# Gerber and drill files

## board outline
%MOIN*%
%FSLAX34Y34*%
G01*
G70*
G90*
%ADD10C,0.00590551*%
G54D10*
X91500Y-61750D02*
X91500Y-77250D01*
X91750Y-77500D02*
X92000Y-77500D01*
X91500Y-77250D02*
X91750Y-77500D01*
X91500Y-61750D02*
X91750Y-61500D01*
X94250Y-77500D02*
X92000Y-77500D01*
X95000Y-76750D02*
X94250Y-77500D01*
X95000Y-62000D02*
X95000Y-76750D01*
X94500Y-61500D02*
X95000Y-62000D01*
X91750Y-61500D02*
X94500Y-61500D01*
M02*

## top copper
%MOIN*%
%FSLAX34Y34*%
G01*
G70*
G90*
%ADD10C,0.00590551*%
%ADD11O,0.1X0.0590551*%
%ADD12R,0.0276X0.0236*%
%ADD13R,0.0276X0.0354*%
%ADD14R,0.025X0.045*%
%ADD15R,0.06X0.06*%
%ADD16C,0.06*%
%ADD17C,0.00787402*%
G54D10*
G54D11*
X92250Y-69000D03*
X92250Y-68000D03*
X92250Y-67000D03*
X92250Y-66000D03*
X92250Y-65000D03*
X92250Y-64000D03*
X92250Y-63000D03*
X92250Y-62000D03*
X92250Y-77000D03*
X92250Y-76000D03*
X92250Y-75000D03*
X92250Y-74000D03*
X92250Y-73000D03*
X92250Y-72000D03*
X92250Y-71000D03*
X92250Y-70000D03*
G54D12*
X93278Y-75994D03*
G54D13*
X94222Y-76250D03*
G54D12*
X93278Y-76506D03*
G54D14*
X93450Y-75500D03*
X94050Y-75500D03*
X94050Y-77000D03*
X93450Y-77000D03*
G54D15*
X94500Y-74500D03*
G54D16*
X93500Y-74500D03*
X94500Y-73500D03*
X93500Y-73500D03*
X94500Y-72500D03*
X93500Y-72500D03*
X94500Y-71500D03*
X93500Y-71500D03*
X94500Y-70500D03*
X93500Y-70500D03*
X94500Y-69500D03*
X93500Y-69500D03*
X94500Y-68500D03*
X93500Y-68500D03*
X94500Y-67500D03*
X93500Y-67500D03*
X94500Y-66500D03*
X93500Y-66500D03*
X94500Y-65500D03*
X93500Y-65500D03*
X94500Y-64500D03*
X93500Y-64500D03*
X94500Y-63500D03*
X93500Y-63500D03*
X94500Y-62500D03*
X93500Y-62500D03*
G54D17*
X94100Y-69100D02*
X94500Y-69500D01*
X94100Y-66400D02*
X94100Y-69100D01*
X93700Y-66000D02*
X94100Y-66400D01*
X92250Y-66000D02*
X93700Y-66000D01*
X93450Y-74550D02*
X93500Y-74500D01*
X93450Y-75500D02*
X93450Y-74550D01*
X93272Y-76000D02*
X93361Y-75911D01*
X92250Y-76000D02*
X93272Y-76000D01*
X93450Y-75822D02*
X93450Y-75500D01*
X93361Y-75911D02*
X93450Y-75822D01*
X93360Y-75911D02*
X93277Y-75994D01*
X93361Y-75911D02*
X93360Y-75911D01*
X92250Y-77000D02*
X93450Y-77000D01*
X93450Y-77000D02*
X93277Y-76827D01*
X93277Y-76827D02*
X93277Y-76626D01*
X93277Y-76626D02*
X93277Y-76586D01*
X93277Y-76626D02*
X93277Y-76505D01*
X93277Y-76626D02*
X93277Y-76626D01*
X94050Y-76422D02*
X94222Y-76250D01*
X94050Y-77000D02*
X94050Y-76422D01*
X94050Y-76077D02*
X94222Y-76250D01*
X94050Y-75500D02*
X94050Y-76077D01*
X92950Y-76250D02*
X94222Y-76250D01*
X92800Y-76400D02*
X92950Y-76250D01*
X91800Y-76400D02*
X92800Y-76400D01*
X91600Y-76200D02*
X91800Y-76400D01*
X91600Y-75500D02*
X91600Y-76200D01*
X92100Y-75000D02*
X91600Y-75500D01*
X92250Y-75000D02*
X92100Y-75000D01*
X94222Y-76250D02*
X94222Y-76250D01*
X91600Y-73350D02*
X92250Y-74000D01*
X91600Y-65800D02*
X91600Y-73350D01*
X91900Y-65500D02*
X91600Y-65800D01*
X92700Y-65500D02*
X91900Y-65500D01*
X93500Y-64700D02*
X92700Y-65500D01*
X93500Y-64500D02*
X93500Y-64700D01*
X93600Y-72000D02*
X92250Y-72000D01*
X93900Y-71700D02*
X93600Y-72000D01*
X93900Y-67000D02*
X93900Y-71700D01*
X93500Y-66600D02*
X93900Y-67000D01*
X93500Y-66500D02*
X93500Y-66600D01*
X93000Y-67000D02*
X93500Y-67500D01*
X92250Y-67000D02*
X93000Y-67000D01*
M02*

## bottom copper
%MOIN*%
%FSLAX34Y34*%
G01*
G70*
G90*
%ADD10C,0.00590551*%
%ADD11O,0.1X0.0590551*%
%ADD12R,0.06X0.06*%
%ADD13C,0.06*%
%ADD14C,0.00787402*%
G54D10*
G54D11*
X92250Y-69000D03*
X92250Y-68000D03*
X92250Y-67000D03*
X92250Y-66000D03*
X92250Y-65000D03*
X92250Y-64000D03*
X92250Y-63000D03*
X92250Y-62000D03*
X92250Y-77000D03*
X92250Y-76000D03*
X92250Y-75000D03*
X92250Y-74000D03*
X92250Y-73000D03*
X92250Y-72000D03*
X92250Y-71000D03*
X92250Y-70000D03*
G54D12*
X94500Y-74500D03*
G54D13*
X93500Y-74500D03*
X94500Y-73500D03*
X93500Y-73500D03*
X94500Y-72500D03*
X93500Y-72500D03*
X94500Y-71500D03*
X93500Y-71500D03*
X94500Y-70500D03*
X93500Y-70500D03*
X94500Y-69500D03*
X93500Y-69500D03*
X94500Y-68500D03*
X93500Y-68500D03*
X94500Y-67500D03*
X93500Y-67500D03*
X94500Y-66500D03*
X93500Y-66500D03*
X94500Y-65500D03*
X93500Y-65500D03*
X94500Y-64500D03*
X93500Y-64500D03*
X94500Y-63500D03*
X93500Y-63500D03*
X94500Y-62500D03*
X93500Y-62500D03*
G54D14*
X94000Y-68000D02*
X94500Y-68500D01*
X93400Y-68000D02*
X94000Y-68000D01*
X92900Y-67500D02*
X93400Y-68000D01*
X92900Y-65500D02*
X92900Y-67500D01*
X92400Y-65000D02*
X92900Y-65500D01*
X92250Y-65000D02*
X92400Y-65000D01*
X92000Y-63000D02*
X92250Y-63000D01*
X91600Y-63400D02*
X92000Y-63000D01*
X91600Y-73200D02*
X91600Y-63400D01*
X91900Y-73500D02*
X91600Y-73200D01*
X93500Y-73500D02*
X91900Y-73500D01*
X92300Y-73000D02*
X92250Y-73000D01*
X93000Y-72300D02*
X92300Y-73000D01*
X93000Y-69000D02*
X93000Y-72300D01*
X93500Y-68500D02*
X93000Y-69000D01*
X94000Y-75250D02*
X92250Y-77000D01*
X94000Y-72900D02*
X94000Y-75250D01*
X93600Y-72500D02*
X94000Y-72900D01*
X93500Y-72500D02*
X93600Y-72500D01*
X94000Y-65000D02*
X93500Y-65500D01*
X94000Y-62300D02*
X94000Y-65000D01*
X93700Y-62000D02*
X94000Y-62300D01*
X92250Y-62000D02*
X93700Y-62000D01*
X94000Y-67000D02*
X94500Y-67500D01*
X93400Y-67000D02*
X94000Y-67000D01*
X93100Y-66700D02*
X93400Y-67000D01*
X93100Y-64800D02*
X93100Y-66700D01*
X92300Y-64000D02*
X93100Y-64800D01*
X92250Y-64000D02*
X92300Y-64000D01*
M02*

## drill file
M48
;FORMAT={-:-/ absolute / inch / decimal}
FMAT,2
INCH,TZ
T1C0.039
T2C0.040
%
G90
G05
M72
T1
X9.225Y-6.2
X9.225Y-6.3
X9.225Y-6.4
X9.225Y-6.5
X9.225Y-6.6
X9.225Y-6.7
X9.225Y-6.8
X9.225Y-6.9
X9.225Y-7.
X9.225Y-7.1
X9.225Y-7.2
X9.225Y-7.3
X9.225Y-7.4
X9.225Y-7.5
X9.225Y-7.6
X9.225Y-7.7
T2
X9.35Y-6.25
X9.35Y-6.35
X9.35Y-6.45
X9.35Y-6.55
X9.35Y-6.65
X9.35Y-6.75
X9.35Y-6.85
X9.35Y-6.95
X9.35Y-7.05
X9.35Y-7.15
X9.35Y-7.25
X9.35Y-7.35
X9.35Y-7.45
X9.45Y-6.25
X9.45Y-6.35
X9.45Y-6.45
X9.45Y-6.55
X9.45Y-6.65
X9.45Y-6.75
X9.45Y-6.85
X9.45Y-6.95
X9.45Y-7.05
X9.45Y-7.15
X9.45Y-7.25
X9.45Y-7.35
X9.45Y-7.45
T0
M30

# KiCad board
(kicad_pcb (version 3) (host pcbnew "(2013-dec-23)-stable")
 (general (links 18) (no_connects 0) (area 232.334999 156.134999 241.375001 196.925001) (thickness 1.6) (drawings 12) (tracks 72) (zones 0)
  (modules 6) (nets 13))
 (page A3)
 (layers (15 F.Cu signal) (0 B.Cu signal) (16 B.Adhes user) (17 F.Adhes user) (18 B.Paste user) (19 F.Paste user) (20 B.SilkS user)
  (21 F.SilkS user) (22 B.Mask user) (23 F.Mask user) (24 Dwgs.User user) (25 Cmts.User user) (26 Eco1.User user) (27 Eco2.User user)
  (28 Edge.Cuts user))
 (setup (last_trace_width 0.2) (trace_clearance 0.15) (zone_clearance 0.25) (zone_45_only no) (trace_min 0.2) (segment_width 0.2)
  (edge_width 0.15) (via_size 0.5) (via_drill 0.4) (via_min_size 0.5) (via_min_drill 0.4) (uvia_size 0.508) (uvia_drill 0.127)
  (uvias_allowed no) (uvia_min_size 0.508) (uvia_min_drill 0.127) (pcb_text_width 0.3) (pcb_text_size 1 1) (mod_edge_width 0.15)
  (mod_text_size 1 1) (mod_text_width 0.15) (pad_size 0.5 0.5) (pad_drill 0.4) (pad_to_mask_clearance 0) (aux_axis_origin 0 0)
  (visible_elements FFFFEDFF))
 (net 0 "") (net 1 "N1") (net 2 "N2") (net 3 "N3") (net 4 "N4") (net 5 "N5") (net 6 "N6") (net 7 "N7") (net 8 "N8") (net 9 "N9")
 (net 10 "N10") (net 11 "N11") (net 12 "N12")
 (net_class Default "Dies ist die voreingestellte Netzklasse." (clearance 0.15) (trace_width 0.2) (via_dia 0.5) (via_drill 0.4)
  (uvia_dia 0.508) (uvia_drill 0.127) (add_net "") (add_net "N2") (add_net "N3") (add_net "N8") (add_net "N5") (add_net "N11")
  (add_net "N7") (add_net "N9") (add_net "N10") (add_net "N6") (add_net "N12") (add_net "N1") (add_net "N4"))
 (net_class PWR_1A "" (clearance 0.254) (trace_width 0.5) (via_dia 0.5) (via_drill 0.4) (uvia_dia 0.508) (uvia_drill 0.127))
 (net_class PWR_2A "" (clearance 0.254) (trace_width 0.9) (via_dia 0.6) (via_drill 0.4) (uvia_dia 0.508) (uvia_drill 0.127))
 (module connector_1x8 (layer F.Cu) (at 234.315 166.37 90)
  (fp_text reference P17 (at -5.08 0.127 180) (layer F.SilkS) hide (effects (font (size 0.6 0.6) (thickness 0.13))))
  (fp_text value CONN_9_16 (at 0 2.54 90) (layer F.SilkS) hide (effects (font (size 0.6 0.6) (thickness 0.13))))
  (pad 1 thru_hole oval (at -8.89 0 90) (size 1.5 2.54) (drill 1) (layers *.Cu *.Mask F.SilkS))
  (pad 2 thru_hole oval (at -6.35 0 90) (size 1.5 2.54) (drill 1) (layers *.Cu *.Mask F.SilkS))
  (pad 3 thru_hole oval (at -3.81 0 90) (size 1.5 2.54) (drill 1) (layers *.Cu *.Mask F.SilkS) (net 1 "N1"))
  (pad 4 thru_hole oval (at -1.27 0 90) (size 1.5 2.54) (drill 1) (layers *.Cu *.Mask F.SilkS) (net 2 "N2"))
  (pad 5 thru_hole oval (at 1.27 0 90) (size 1.5 2.54) (drill 1) (layers *.Cu *.Mask F.SilkS) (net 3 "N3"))
  (pad 6 thru_hole oval (at 3.81 0 90) (size 1.5 2.54) (drill 1) (layers *.Cu *.Mask F.SilkS) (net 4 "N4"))
  (pad 7 thru_hole oval (at 6.35 0 90) (size 1.5 2.54) (drill 1) (layers *.Cu *.Mask F.SilkS) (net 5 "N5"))
  (pad 8 thru_hole oval (at 8.89 0 90) (size 1.5 2.54) (drill 1) (layers *.Cu *.Mask F.SilkS) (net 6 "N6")))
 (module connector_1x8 (layer F.Cu) (at 234.315 186.69 90)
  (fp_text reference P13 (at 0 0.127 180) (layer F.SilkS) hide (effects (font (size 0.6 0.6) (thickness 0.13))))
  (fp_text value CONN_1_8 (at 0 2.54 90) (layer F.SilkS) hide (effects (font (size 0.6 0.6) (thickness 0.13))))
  (pad 1 thru_hole oval (at -8.89 0 90) (size 1.5 2.54) (drill 1) (layers *.Cu *.Mask F.SilkS) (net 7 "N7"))
  (pad 2 thru_hole oval (at -6.35 0 90) (size 1.5 2.54) (drill 1) (layers *.Cu *.Mask F.SilkS) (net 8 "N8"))
  (pad 3 thru_hole oval (at -3.81 0 90) (size 1.5 2.54) (drill 1) (layers *.Cu *.Mask F.SilkS) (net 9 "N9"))
  (pad 4 thru_hole oval (at -1.27 0 90) (size 1.5 2.54) (drill 1) (layers *.Cu *.Mask F.SilkS) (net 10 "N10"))
  (pad 5 thru_hole oval (at 1.27 0 90) (size 1.5 2.54) (drill 1) (layers *.Cu *.Mask F.SilkS) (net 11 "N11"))
  (pad 6 thru_hole oval (at 3.81 0 90) (size 1.5 2.54) (drill 1) (layers *.Cu *.Mask F.SilkS) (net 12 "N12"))
  (pad 7 thru_hole oval (at 6.35 0 90) (size 1.5 2.54) (drill 1) (layers *.Cu *.Mask F.SilkS))
  (pad 8 thru_hole oval (at 8.89 0 90) (size 1.5 2.54) (drill 1) (layers *.Cu *.Mask F.SilkS)))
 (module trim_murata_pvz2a (layer F.Cu) (at 238.125 193.675 270)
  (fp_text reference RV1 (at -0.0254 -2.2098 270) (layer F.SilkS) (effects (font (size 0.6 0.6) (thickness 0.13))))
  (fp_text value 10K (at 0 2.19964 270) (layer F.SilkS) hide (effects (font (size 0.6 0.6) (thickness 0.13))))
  (pad 1 smd rect (at -0.65024 1.19888 270) (size 0.59944 0.70104) (layers F.Cu F.Paste F.Mask) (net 8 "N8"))
  (pad 2 smd rect (at 0 -1.19888 270) (size 0.89916 0.70104) (layers F.Cu F.Paste F.Mask) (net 9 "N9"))
  (pad 3 smd rect (at 0.65024 1.19888 270) (size 0.59944 0.70104) (layers F.Cu F.Paste F.Mask) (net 7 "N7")))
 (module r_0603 (layer F.Cu) (at 238.125 191.77)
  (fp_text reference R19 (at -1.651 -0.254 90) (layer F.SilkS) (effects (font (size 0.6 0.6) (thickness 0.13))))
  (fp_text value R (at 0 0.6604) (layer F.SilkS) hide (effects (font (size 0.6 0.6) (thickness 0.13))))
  (pad 1 smd rect (at -0.762 0) (size 0.635 1.143) (layers F.Cu F.Paste F.Mask) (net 8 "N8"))
  (pad 2 smd rect (at 0.762 0) (size 0.635 1.143) (layers F.Cu F.Paste F.Mask) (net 9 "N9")))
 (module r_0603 (layer F.Cu) (at 238.125 195.58 180)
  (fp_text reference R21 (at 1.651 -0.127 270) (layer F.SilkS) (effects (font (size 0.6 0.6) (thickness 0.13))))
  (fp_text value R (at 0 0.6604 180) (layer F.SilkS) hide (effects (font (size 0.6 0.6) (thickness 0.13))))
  (pad 1 smd rect (at -0.762 0 180) (size 0.635 1.143) (layers F.Cu F.Paste F.Mask) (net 9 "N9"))
  (pad 2 smd rect (at 0.762 0 180) (size 0.635 1.143) (layers F.Cu F.Paste F.Mask) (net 7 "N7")))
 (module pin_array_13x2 (layer F.Cu) (at 238.76 173.99 90)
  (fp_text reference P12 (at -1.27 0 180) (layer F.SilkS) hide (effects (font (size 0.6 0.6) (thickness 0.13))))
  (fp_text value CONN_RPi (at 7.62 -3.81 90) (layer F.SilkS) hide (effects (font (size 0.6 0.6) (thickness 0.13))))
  (pad 1 thru_hole rect (at -15.24 1.27 90) (size 1.524 1.524) (drill 1.016) (layers *.Cu *.Mask F.SilkS))
  (pad 2 thru_hole circle (at -15.24 -1.27 90) (size 1.524 1.524) (drill 1.016) (layers *.Cu *.Mask F.SilkS) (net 8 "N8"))
  (pad 3 thru_hole circle (at -12.7 1.27 90) (size 1.524 1.524) (drill 1.016) (layers *.Cu *.Mask F.SilkS))
  (pad 4 thru_hole circle (at -12.7 -1.27 90) (size 1.524 1.524) (drill 1.016) (layers *.Cu *.Mask F.SilkS) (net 5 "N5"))
  (pad 5 thru_hole circle (at -10.16 1.27 90) (size 1.524 1.524) (drill 1.016) (layers *.Cu *.Mask F.SilkS))
  (pad 6 thru_hole circle (at -10.16 -1.27 90) (size 1.524 1.524) (drill 1.016) (layers *.Cu *.Mask F.SilkS) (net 7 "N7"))
  (pad 7 thru_hole circle (at -7.62 1.27 90) (size 1.524 1.524) (drill 1.016) (layers *.Cu *.Mask F.SilkS))
  (pad 8 thru_hole circle (at -7.62 -1.27 90) (size 1.524 1.524) (drill 1.016) (layers *.Cu *.Mask F.SilkS))
  (pad 9 thru_hole circle (at -5.08 1.27 90) (size 1.524 1.524) (drill 1.016) (layers *.Cu *.Mask F.SilkS))
  (pad 10 thru_hole circle (at -5.08 -1.27 90) (size 1.524 1.524) (drill 1.016) (layers *.Cu *.Mask F.SilkS))
  (pad 11 thru_hole circle (at -2.54 1.27 90) (size 1.524 1.524) (drill 1.016) (layers *.Cu *.Mask F.SilkS) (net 2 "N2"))
  (pad 12 thru_hole circle (at -2.54 -1.27 90) (size 1.524 1.524) (drill 1.016) (layers *.Cu *.Mask F.SilkS))
  (pad 13 thru_hole circle (at 0 1.27 90) (size 1.524 1.524) (drill 1.016) (layers *.Cu *.Mask F.SilkS) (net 3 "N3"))
  (pad 14 thru_hole circle (at 0 -1.27 90) (size 1.524 1.524) (drill 1.016) (layers *.Cu *.Mask F.SilkS) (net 11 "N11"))
  (pad 15 thru_hole circle (at 2.54 1.27 90) (size 1.524 1.524) (drill 1.016) (layers *.Cu *.Mask F.SilkS) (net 4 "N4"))
  (pad 16 thru_hole circle (at 2.54 -1.27 90) (size 1.524 1.524) (drill 1.016) (layers *.Cu *.Mask F.SilkS) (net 1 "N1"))
  (pad 17 thru_hole circle (at 5.08 1.27 90) (size 1.524 1.524) (drill 1.016) (layers *.Cu *.Mask F.SilkS))
  (pad 18 thru_hole circle (at 5.08 -1.27 90) (size 1.524 1.524) (drill 1.016) (layers *.Cu *.Mask F.SilkS) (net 12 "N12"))
  (pad 19 thru_hole circle (at 7.62 1.27 90) (size 1.524 1.524) (drill 1.016) (layers *.Cu *.Mask F.SilkS))
  (pad 20 thru_hole circle (at 7.62 -1.27 90) (size 1.524 1.524) (drill 1.016) (layers *.Cu *.Mask F.SilkS) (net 6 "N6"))
  (pad 21 thru_hole circle (at 10.16 1.27 90) (size 1.524 1.524) (drill 1.016) (layers *.Cu *.Mask F.SilkS))
  (pad 22 thru_hole circle (at 10.16 -1.27 90) (size 1.524 1.524) (drill 1.016) (layers *.Cu *.Mask F.SilkS) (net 10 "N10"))
  (pad 23 thru_hole circle (at 12.7 1.27 90) (size 1.524 1.524) (drill 1.016) (layers *.Cu *.Mask F.SilkS))
  (pad 24 thru_hole circle (at 12.7 -1.27 90) (size 1.524 1.524) (drill 1.016) (layers *.Cu *.Mask F.SilkS))
  (pad 25 thru_hole circle (at 15.24 1.27 90) (size 1.524 1.524) (drill 1.016) (layers *.Cu *.Mask F.SilkS))
  (pad 26 thru_hole circle (at 15.24 -1.27 90) (size 1.524 1.524) (drill 1.016) (layers *.Cu *.Mask F.SilkS)))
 (gr_line (start 232.41 156.845) (end 232.41 196.215) (angle 90) (layer Edge.Cuts) (width 0.15))
 (gr_line (start 233.045 196.85) (end 233.68 196.85) (angle 90) (layer Edge.Cuts) (width 0.15))
 (gr_line (start 232.41 196.215) (end 233.045 196.85) (angle 90) (layer Edge.Cuts) (width 0.15))
 (gr_line (start 232.41 156.845) (end 233.045 156.21) (angle 90) (layer Edge.Cuts) (width 0.15))
 (gr_line (start 239.395 196.85) (end 233.68 196.85) (angle 90) (layer Edge.Cuts) (width 0.15))
 (gr_line (start 241.3 194.945) (end 239.395 196.85) (angle 90) (layer Edge.Cuts) (width 0.15))
 (gr_line (start 241.3 157.48) (end 241.3 194.945) (angle 90) (layer Edge.Cuts) (width 0.15))
 (gr_line (start 240.03 156.21) (end 241.3 157.48) (angle 90) (layer Edge.Cuts) (width 0.15))
 (gr_line (start 233.045 156.21) (end 240.03 156.21) (angle 90) (layer Edge.Cuts) (width 0.15))
 (segment (start 239.014 175.514) (end 240.03 176.53) (width 0.2) (layer F.Cu) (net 2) (status 20))
 (segment (start 239.014 168.656) (end 239.014 175.514) (width 0.2) (layer F.Cu) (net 2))
 (segment (start 237.998 167.64) (end 239.014 168.656) (width 0.2) (layer F.Cu) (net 2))
 (segment (start 234.315 167.64) (end 237.998 167.64) (width 0.2) (layer F.Cu) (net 2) (status 10))
 (segment (start 238.76 172.72) (end 240.03 173.99) (width 0.2) (layer B.Cu) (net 3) (status 20))
 (segment (start 237.236 172.72) (end 238.76 172.72) (width 0.2) (layer B.Cu) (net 3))
 (segment (start 235.966 171.45) (end 237.236 172.72) (width 0.2) (layer B.Cu) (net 3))
 (segment (start 235.966 166.37) (end 235.966 171.45) (width 0.2) (layer B.Cu) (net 3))
 (segment (start 234.696 165.1) (end 235.966 166.37) (width 0.2) (layer B.Cu) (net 3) (status 10))
 (segment (start 234.315 165.1) (end 234.696 165.1) (width 0.2) (layer B.Cu) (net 3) (status 30))
 (segment (start 237.363 189.357) (end 237.49 189.23) (width 0.2) (layer F.Cu) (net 8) (status 30))
 (segment (start 237.363 191.77) (end 237.363 189.357) (width 0.2) (layer F.Cu) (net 8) (status 30))
 (segment (start 236.911 193.04) (end 237.137 192.814) (width 0.2) (layer F.Cu) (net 8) (status 30))
 (segment (start 234.315 193.04) (end 236.911 193.04) (width 0.2) (layer F.Cu) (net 8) (status 30))
 (segment (start 237.363 192.588) (end 237.363 191.77) (width 0.2) (layer F.Cu) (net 8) (status 20))
 (segment (start 237.137 192.814) (end 237.363 192.588) (width 0.2) (layer F.Cu) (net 8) (status 10))
 (segment (start 237.1369 192.814) (end 236.9261 193.0248) (width 0.2) (layer F.Cu) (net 8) (status 30))
 (segment (start 237.137 192.814) (end 237.1369 192.814) (width 0.2) (layer F.Cu) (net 8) (status 30))
 (segment (start 233.68 160.02) (end 234.315 160.02) (width 0.2) (layer B.Cu) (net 5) (status 30))
 (segment (start 232.664 161.036) (end 233.68 160.02) (width 0.2) (layer B.Cu) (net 5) (status 20))
 (segment (start 232.664 185.928) (end 232.664 161.036) (width 0.2) (layer B.Cu) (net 5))
 (segment (start 233.426 186.69) (end 232.664 185.928) (width 0.2) (layer B.Cu) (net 5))
 (segment (start 237.49 186.69) (end 233.426 186.69) (width 0.2) (layer B.Cu) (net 5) (status 10))
 (segment (start 234.442 185.42) (end 234.315 185.42) (width 0.2) (layer B.Cu) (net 11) (status 30))
 (segment (start 236.22 183.642) (end 234.442 185.42) (width 0.2) (layer B.Cu) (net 11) (status 20))
 (segment (start 236.22 175.26) (end 236.22 183.642) (width 0.2) (layer B.Cu) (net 11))
 (segment (start 237.49 173.99) (end 236.22 175.26) (width 0.2) (layer B.Cu) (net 11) (status 10))
 (segment (start 238.76 191.135) (end 234.315 195.58) (width 0.2) (layer B.Cu) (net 7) (status 20))
 (segment (start 238.76 185.166) (end 238.76 191.135) (width 0.2) (layer B.Cu) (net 7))
 (segment (start 237.744 184.15) (end 238.76 185.166) (width 0.2) (layer B.Cu) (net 7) (status 10))
 (segment (start 237.49 184.15) (end 237.744 184.15) (width 0.2) (layer B.Cu) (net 7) (status 30))
 (segment (start 234.315 195.58) (end 237.363 195.58) (width 0.2) (layer F.Cu) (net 7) (status 30))
 (segment (start 237.363 195.58) (end 236.926 195.143) (width 0.2) (layer F.Cu) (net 7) (status 10))
 (segment (start 236.926 195.143) (end 236.926 194.632) (width 0.2) (layer F.Cu) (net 7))
 (segment (start 236.926 194.632) (end 236.926 194.53) (width 0.2) (layer F.Cu) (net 7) (status 20))
 (segment (start 236.9261 194.6319) (end 236.9261 194.3252) (width 0.2) (layer F.Cu) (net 7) (status 20))
 (segment (start 236.926 194.632) (end 236.9261 194.6319) (width 0.2) (layer F.Cu) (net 7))
 (segment (start 238.887 194.112) (end 239.324 193.675) (width 0.2) (layer F.Cu) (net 9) (status 20))
 (segment (start 238.887 195.58) (end 238.887 194.112) (width 0.2) (layer F.Cu) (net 9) (status 10))
 (segment (start 238.887 193.238) (end 239.324 193.675) (width 0.2) (layer F.Cu) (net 9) (status 20))
 (segment (start 238.887 191.77) (end 238.887 193.238) (width 0.2) (layer F.Cu) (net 9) (status 10))
 (segment (start 236.093 193.675) (end 239.3239 193.675) (width 0.2) (layer F.Cu) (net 9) (status 20))
 (segment (start 235.712 194.056) (end 236.093 193.675) (width 0.2) (layer F.Cu) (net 9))
 (segment (start 233.172 194.056) (end 235.712 194.056) (width 0.2) (layer F.Cu) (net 9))
 (segment (start 232.664 193.548) (end 233.172 194.056) (width 0.2) (layer F.Cu) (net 9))
 (segment (start 232.664 191.77) (end 232.664 193.548) (width 0.2) (layer F.Cu) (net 9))
 (segment (start 233.934 190.5) (end 232.664 191.77) (width 0.2) (layer F.Cu) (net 9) (status 10))
 (segment (start 234.315 190.5) (end 233.934 190.5) (width 0.2) (layer F.Cu) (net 9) (status 30))
 (segment (start 239.3239 193.675) (end 239.324 193.675) (width 0.2) (layer F.Cu) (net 9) (status 30))
 (segment (start 232.664 186.309) (end 234.315 187.96) (width 0.2) (layer F.Cu) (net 10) (status 20))
 (segment (start 232.664 167.132) (end 232.664 186.309) (width 0.2) (layer F.Cu) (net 10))
 (segment (start 233.426 166.37) (end 232.664 167.132) (width 0.2) (layer F.Cu) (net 10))
 (segment (start 235.458 166.37) (end 233.426 166.37) (width 0.2) (layer F.Cu) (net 10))
 (segment (start 237.49 164.338) (end 235.458 166.37) (width 0.2) (layer F.Cu) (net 10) (status 10))
 (segment (start 237.49 163.83) (end 237.49 164.338) (width 0.2) (layer F.Cu) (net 10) (status 30))
 (segment (start 238.76 165.1) (end 237.49 166.37) (width 0.2) (layer B.Cu) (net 6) (status 20))
 (segment (start 238.76 158.242) (end 238.76 165.1) (width 0.2) (layer B.Cu) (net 6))
 (segment (start 237.998 157.48) (end 238.76 158.242) (width 0.2) (layer B.Cu) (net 6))
 (segment (start 234.315 157.48) (end 237.998 157.48) (width 0.2) (layer B.Cu) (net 6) (status 10))
 (segment (start 237.744 182.88) (end 234.315 182.88) (width 0.2) (layer F.Cu) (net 12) (status 20))
 (segment (start 238.506 182.118) (end 237.744 182.88) (width 0.2) (layer F.Cu) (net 12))
 (segment (start 238.506 170.18) (end 238.506 182.118) (width 0.2) (layer F.Cu) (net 12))
 (segment (start 237.49 169.164) (end 238.506 170.18) (width 0.2) (layer F.Cu) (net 12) (status 10))
 (segment (start 237.49 168.91) (end 237.49 169.164) (width 0.2) (layer F.Cu) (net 12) (status 30))
 (segment (start 236.22 170.18) (end 237.49 171.45) (width 0.2) (layer F.Cu) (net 1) (status 20))
 (segment (start 234.315 170.18) (end 236.22 170.18) (width 0.2) (layer F.Cu) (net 1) (status 10))
 (segment (start 238.76 170.18) (end 240.03 171.45) (width 0.2) (layer B.Cu) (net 4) (status 20))
 (segment (start 237.236 170.18) (end 238.76 170.18) (width 0.2) (layer B.Cu) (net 4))
 (segment (start 236.474 169.418) (end 237.236 170.18) (width 0.2) (layer B.Cu) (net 4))
 (segment (start 236.474 164.592) (end 236.474 169.418) (width 0.2) (layer B.Cu) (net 4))
 (segment (start 234.442 162.56) (end 236.474 164.592) (width 0.2) (layer B.Cu) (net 4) (status 10))
 (segment (start 234.315 162.56) (end 234.442 162.56) (width 0.2) (layer B.Cu) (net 4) (status 30)))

